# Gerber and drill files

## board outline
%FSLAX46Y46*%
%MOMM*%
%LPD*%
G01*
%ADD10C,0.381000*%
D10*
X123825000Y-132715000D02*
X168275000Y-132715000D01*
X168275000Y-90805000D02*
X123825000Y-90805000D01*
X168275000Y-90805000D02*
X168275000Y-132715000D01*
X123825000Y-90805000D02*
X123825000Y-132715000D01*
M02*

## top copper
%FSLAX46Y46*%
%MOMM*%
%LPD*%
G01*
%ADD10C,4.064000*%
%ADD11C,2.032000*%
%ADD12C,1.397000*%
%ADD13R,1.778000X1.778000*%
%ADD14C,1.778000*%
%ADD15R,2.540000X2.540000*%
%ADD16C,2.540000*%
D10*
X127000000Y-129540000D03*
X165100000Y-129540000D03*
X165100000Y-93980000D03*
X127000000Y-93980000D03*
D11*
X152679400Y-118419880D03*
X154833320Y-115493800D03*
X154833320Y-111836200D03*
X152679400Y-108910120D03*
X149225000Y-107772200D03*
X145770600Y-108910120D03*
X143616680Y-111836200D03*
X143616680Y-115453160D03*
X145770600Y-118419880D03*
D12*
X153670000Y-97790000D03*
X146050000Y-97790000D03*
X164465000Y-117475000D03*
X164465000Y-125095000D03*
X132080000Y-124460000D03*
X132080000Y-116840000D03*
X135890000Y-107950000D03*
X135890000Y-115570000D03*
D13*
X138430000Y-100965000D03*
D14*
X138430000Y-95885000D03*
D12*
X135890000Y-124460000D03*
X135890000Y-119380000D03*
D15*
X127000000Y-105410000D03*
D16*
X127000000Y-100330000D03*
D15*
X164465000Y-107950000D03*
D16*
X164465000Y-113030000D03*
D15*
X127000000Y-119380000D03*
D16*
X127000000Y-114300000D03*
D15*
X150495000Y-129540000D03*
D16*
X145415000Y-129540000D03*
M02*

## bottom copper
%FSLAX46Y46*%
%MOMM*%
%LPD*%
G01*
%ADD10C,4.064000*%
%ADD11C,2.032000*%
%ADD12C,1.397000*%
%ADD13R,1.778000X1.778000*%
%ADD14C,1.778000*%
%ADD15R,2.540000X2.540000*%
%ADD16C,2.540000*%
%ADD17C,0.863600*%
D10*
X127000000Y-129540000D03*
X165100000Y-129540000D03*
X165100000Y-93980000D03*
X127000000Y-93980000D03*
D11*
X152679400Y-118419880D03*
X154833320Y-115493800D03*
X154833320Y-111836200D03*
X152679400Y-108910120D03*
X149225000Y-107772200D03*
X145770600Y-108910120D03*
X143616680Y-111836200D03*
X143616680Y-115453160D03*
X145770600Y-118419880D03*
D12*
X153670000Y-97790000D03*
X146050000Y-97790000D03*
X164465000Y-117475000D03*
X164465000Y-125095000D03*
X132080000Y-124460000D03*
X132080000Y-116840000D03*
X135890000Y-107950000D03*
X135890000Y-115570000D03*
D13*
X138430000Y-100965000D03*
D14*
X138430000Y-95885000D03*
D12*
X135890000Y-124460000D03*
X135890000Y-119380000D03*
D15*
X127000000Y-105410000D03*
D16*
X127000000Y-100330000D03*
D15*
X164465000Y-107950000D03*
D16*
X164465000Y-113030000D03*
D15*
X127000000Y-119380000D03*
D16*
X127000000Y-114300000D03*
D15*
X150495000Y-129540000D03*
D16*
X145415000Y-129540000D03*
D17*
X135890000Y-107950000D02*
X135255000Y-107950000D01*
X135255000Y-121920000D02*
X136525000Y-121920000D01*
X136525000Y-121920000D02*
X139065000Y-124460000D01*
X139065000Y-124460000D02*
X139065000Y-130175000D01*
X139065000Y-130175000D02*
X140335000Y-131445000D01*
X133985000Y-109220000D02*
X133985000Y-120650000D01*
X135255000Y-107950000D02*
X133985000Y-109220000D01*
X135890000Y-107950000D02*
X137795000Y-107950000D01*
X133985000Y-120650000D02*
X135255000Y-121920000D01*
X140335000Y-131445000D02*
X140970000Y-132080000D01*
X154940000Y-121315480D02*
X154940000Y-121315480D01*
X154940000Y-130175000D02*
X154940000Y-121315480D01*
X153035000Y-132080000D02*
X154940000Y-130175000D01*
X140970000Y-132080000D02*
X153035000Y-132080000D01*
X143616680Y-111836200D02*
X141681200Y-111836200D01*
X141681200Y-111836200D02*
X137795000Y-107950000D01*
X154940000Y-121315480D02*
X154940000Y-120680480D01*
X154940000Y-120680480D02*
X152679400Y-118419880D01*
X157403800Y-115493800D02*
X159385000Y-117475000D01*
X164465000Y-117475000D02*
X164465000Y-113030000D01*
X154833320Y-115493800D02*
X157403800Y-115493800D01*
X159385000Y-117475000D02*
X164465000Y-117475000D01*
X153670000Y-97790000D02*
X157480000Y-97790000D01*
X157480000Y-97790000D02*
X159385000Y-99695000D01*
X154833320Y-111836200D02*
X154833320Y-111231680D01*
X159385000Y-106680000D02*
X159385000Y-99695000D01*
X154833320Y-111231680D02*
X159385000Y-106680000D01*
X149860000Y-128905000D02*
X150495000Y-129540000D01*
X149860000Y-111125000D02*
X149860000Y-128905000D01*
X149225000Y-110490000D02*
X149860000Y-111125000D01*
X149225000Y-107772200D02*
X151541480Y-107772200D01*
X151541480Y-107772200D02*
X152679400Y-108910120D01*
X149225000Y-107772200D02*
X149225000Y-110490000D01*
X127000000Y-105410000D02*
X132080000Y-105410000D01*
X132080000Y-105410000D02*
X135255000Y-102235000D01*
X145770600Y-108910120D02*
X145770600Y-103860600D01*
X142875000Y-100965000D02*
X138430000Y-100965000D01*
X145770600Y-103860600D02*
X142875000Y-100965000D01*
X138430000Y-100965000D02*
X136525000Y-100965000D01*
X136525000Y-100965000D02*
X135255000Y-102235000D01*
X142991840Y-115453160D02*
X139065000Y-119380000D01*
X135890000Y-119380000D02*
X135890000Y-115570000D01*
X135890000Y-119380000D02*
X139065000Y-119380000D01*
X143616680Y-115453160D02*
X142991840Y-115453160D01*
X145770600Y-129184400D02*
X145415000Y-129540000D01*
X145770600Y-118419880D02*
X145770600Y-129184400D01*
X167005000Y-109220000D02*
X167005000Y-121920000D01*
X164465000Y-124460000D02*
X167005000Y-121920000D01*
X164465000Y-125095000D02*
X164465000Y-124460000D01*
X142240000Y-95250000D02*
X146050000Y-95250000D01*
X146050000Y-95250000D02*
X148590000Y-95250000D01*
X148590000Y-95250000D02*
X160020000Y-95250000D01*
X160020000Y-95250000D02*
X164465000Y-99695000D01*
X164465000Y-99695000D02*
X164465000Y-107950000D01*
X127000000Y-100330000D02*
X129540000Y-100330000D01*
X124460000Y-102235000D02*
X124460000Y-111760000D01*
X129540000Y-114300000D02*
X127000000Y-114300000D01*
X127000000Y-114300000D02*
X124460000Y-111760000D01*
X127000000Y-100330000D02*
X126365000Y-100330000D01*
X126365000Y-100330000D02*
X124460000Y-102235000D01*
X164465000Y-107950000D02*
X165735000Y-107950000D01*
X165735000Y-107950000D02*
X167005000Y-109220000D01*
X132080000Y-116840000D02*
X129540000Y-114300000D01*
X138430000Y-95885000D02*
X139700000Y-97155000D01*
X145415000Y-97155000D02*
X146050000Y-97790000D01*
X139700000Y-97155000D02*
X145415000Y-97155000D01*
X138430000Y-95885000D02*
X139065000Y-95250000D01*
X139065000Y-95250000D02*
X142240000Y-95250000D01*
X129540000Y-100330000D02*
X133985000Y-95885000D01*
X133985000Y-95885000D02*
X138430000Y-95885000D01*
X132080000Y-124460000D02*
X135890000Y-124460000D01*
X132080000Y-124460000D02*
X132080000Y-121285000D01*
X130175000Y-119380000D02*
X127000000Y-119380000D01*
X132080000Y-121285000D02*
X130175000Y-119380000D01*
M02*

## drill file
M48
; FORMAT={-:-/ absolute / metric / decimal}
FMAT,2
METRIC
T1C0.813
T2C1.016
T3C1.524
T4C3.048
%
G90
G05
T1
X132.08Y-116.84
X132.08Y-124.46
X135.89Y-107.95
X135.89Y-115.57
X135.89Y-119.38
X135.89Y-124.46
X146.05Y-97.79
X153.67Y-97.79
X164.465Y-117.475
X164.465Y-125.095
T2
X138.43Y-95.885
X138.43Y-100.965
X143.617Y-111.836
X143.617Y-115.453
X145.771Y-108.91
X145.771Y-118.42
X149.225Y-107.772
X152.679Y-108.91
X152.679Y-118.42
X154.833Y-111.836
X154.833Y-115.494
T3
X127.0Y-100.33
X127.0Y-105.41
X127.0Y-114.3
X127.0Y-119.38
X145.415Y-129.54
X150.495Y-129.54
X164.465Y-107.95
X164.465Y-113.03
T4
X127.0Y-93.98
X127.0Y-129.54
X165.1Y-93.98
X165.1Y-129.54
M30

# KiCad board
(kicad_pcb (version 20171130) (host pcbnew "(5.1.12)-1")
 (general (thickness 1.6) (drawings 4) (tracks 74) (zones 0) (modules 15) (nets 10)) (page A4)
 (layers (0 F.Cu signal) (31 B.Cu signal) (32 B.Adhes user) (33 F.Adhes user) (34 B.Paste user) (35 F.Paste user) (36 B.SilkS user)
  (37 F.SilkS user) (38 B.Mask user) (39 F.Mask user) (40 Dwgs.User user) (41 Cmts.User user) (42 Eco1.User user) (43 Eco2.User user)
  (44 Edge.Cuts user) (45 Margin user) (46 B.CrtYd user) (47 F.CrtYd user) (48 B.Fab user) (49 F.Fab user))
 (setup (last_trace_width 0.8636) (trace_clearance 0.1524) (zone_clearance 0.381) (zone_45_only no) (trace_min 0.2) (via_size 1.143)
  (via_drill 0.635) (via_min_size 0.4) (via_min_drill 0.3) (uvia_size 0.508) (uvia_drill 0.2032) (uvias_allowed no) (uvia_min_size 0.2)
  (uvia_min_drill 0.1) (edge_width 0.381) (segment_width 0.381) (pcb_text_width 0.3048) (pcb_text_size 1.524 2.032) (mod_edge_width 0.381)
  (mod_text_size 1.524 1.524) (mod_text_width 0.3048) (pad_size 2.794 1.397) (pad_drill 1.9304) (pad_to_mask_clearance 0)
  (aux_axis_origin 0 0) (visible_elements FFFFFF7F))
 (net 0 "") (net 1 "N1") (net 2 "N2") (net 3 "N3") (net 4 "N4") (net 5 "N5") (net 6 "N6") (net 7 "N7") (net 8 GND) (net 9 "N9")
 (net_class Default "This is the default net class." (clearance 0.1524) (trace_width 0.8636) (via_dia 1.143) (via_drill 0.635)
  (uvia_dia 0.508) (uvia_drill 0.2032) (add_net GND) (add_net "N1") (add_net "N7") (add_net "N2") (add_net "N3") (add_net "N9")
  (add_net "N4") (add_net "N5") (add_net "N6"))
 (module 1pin (layer F.Cu) (at 127 129.54)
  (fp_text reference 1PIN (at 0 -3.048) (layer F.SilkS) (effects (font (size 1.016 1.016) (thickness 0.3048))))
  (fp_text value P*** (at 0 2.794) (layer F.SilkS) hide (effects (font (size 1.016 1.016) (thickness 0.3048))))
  (pad 1 thru_hole circle (at 0 0) (size 4.064 4.064) (drill 3.048) (layers *.Cu *.Mask F.SilkS)))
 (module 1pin (layer F.Cu) (at 165.1 129.54)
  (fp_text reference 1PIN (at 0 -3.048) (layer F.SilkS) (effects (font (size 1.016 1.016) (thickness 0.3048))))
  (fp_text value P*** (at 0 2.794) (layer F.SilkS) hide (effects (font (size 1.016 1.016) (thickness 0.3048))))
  (pad 1 thru_hole circle (at 0 0) (size 4.064 4.064) (drill 3.048) (layers *.Cu *.Mask F.SilkS)))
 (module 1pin (layer F.Cu) (at 165.1 93.98)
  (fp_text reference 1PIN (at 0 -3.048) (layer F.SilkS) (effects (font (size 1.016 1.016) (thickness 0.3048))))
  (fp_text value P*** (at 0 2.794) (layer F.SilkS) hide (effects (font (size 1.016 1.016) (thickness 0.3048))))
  (pad 1 thru_hole circle (at 0 0) (size 4.064 4.064) (drill 3.048) (layers *.Cu *.Mask F.SilkS)))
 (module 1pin (layer F.Cu) (at 127 93.98)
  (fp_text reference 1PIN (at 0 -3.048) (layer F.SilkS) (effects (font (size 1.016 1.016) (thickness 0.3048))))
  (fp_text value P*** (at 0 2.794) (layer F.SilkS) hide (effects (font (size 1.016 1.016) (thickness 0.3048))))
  (pad 1 thru_hole circle (at 0 0) (size 4.064 4.064) (drill 3.048) (layers *.Cu *.Mask F.SilkS)))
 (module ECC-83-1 (layer F.Cu) (at 149.225 113.665)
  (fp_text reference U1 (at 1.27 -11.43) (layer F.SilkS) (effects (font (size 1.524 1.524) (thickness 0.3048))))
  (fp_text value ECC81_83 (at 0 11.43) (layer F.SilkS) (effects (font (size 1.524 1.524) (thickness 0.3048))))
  (pad 1 thru_hole circle (at 3.4544 4.75488) (size 2.032 2.032) (drill 1.016) (layers *.Cu *.Mask F.SilkS) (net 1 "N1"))
  (pad 2 thru_hole circle (at 5.60832 1.8288) (size 2.032 2.032) (drill 1.016) (layers *.Cu *.Mask F.SilkS) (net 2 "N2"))
  (pad 3 thru_hole circle (at 5.60832 -1.8288) (size 2.032 2.032) (drill 1.016) (layers *.Cu *.Mask F.SilkS) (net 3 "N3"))
  (pad 4 thru_hole circle (at 3.4544 -4.75488) (size 2.032 2.032) (drill 1.016) (layers *.Cu *.Mask F.SilkS) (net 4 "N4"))
  (pad 5 thru_hole circle (at 0 -5.8928) (size 2.032 2.032) (drill 1.016) (layers *.Cu *.Mask F.SilkS) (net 4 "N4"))
  (pad 6 thru_hole circle (at -3.4544 -4.75488) (size 2.032 2.032) (drill 1.016) (layers *.Cu *.Mask F.SilkS) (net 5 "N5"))
  (pad 7 thru_hole circle (at -5.60832 -1.8288) (size 2.032 2.032) (drill 1.016) (layers *.Cu *.Mask F.SilkS) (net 1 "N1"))
  (pad 8 thru_hole circle (at -5.60832 1.78816) (size 2.032 2.032) (drill 1.016) (layers *.Cu *.Mask F.SilkS) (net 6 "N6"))
  (pad 9 thru_hole circle (at -3.4544 4.75488) (size 2.032 2.032) (drill 1.016) (layers *.Cu *.Mask F.SilkS) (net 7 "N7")))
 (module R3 (layer F.Cu) (at 149.86 97.79 180) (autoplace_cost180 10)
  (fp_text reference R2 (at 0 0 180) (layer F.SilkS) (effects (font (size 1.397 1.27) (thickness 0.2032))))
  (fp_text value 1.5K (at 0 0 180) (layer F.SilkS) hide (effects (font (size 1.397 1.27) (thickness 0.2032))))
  (pad 1 thru_hole circle (at -3.81 0 180) (size 1.397 1.397) (drill 0.8128) (layers *.Cu *.Mask F.SilkS) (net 3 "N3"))
  (pad 2 thru_hole circle (at 3.81 0 180) (size 1.397 1.397) (drill 0.8128) (layers *.Cu *.Mask F.SilkS) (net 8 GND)))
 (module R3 (layer F.Cu) (at 164.465 121.285 270) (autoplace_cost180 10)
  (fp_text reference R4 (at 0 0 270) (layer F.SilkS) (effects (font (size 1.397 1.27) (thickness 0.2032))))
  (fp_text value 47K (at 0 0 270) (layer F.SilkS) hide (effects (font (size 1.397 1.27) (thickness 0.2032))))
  (pad 1 thru_hole circle (at -3.81 0 270) (size 1.397 1.397) (drill 0.8128) (layers *.Cu *.Mask F.SilkS) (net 2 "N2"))
  (pad 2 thru_hole circle (at 3.81 0 270) (size 1.397 1.397) (drill 0.8128) (layers *.Cu *.Mask F.SilkS) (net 8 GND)))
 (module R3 (layer F.Cu) (at 132.08 120.65 90) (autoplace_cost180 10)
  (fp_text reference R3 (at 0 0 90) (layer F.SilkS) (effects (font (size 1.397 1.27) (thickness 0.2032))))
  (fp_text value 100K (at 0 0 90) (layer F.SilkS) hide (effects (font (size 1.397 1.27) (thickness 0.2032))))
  (pad 1 thru_hole circle (at -3.81 0 90) (size 1.397 1.397) (drill 0.8128) (layers *.Cu *.Mask F.SilkS) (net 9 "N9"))
  (pad 2 thru_hole circle (at 3.81 0 90) (size 1.397 1.397) (drill 0.8128) (layers *.Cu *.Mask F.SilkS) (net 8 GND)))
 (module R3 (layer F.Cu) (at 135.89 111.76 270) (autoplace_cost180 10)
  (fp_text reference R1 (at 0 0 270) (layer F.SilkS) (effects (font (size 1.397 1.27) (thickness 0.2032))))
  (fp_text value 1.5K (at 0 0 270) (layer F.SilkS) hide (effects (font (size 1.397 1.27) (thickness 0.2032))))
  (pad 1 thru_hole circle (at -3.81 0 270) (size 1.397 1.397) (drill 0.8128) (layers *.Cu *.Mask F.SilkS) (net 1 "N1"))
  (pad 2 thru_hole circle (at 3.81 0 270) (size 1.397 1.397) (drill 0.8128) (layers *.Cu *.Mask F.SilkS) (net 6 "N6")))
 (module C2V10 (layer F.Cu) (at 138.43 98.425 90)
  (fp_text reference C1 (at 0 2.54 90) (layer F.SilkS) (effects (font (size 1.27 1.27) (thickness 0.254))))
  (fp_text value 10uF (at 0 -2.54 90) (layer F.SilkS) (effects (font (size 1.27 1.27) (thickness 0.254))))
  (pad 1 thru_hole rect (at -2.54 0 90) (size 1.778 1.778) (drill 1.016) (layers *.Cu *.Mask F.SilkS) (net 5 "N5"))
  (pad 2 thru_hole circle (at 2.54 0 90) (size 1.778 1.778) (drill 1.016) (layers *.Cu *.Mask F.SilkS) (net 8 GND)))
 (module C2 (layer F.Cu) (at 135.89 121.92 90)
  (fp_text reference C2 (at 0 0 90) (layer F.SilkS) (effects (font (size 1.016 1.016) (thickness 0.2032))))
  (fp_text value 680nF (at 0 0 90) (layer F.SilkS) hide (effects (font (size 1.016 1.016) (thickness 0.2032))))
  (pad 1 thru_hole circle (at -2.54 0 90) (size 1.397 1.397) (drill 0.8128) (layers *.Cu *.Mask F.SilkS) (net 9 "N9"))
  (pad 2 thru_hole circle (at 2.54 0 90) (size 1.397 1.397) (drill 0.8128) (layers *.Cu *.Mask F.SilkS) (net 6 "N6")))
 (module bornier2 (layer F.Cu) (at 127 102.87 90)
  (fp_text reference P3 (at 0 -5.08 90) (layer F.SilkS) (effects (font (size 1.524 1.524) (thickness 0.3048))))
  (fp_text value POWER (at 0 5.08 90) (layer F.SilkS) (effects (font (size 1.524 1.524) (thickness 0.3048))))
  (pad 1 thru_hole rect (at -2.54 0 90) (size 2.54 2.54) (drill 1.524) (layers *.Cu *.Mask F.SilkS) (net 5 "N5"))
  (pad 2 thru_hole circle (at 2.54 0 90) (size 2.54 2.54) (drill 1.524) (layers *.Cu *.Mask F.SilkS) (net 8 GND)))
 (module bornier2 (layer F.Cu) (at 164.465 110.49 270)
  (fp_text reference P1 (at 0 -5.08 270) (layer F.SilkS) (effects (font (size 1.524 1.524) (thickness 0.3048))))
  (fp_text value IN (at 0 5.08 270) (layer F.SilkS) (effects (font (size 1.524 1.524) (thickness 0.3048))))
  (pad 1 thru_hole rect (at -2.54 0 270) (size 2.54 2.54) (drill 1.524) (layers *.Cu *.Mask F.SilkS) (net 8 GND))
  (pad 2 thru_hole circle (at 2.54 0 270) (size 2.54 2.54) (drill 1.524) (layers *.Cu *.Mask F.SilkS) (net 2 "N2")))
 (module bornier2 (layer F.Cu) (at 127 116.84 90)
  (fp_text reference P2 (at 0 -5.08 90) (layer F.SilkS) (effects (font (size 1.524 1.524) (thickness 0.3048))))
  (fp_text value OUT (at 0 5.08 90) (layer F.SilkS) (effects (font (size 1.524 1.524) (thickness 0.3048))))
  (pad 1 thru_hole rect (at -2.54 0 90) (size 2.54 2.54) (drill 1.524) (layers *.Cu *.Mask F.SilkS) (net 9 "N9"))
  (pad 2 thru_hole circle (at 2.54 0 90) (size 2.54 2.54) (drill 1.524) (layers *.Cu *.Mask F.SilkS) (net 8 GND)))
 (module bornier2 (layer F.Cu) (at 147.955 129.54 180)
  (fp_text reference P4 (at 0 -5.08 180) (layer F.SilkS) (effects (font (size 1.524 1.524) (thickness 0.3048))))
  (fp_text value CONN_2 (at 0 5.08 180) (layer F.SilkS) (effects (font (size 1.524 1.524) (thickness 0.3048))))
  (pad 1 thru_hole rect (at -2.54 0 180) (size 2.54 2.54) (drill 1.524) (layers *.Cu *.Mask F.SilkS) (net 4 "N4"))
  (pad 2 thru_hole circle (at 2.54 0 180) (size 2.54 2.54) (drill 1.524) (layers *.Cu *.Mask F.SilkS) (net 7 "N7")))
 (gr_line (start 123.825 132.715) (end 168.275 132.715) (angle 90) (layer Edge.Cuts) (width 0.381))
 (gr_line (start 168.275 90.805) (end 123.825 90.805) (angle 90) (layer Edge.Cuts) (width 0.381))
 (gr_line (start 168.275 90.805) (end 168.275 132.715) (angle 90) (layer Edge.Cuts) (width 0.381))
 (gr_line (start 123.825 90.805) (end 123.825 132.715) (angle 90) (layer Edge.Cuts) (width 0.381))
 (segment (start 135.89 107.95) (end 135.255 107.95) (width 0.8636) (layer B.Cu) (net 1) (status 800))
 (segment (start 135.255 121.92) (end 136.525 121.92) (width 0.8636) (layer B.Cu) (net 1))
 (segment (start 136.525 121.92) (end 139.065 124.46) (width 0.8636) (layer B.Cu) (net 1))
 (segment (start 139.065 124.46) (end 139.065 130.175) (width 0.8636) (layer B.Cu) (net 1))
 (segment (start 139.065 130.175) (end 140.335 131.445) (width 0.8636) (layer B.Cu) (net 1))
 (segment (start 133.985 109.22) (end 133.985 120.65) (width 0.8636) (layer B.Cu) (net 1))
 (segment (start 135.255 107.95) (end 133.985 109.22) (width 0.8636) (layer B.Cu) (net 1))
 (segment (start 135.89 107.95) (end 137.795 107.95) (width 0.8636) (layer B.Cu) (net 1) (status 800))
 (segment (start 133.985 120.65) (end 135.255 121.92) (width 0.8636) (layer B.Cu) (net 1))
 (segment (start 140.335 131.445) (end 140.97 132.08) (width 0.8636) (layer B.Cu) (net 1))
 (segment (start 154.94 121.31548) (end 154.94 121.31548) (width 0.8636) (layer B.Cu) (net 1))
 (segment (start 154.94 130.175) (end 154.94 121.31548) (width 0.8636) (layer B.Cu) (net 1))
 (segment (start 153.035 132.08) (end 154.94 130.175) (width 0.8636) (layer B.Cu) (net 1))
 (segment (start 140.97 132.08) (end 153.035 132.08) (width 0.8636) (layer B.Cu) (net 1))
 (segment (start 143.61668 111.8362) (end 141.6812 111.8362) (width 0.8636) (layer B.Cu) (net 1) (status 800))
 (segment (start 141.6812 111.8362) (end 137.795 107.95) (width 0.8636) (layer B.Cu) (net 1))
 (segment (start 154.94 121.31548) (end 154.94 120.68048) (width 0.8636) (layer B.Cu) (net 1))
 (segment (start 154.94 120.68048) (end 152.6794 118.41988) (width 0.8636) (layer B.Cu) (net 1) (status 400))
 (segment (start 157.4038 115.4938) (end 159.385 117.475) (width 0.8636) (layer B.Cu) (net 2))
 (segment (start 164.465 117.475) (end 164.465 113.03) (width 0.8636) (layer B.Cu) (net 2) (status C00))
 (segment (start 154.83332 115.4938) (end 157.4038 115.4938) (width 0.8636) (layer B.Cu) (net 2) (status 800))
 (segment (start 159.385 117.475) (end 164.465 117.475) (width 0.8636) (layer B.Cu) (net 2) (status 400))
 (segment (start 153.67 97.79) (end 157.48 97.79) (width 0.8636) (layer B.Cu) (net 3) (status 800))
 (segment (start 157.48 97.79) (end 159.385 99.695) (width 0.8636) (layer B.Cu) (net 3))
 (segment (start 154.83332 111.8362) (end 154.83332 111.23168) (width 0.8636) (layer B.Cu) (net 3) (status 800))
 (segment (start 159.385 106.68) (end 159.385 99.695) (width 0.8636) (layer B.Cu) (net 3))
 (segment (start 154.83332 111.23168) (end 159.385 106.68) (width 0.8636) (layer B.Cu) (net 3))
 (segment (start 149.86 128.905) (end 150.495 129.54) (width 0.8636) (layer B.Cu) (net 4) (status 400))
 (segment (start 149.86 111.125) (end 149.86 128.905) (width 0.8636) (layer B.Cu) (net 4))
 (segment (start 149.225 110.49) (end 149.86 111.125) (width 0.8636) (layer B.Cu) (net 4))
 (segment (start 149.225 107.7722) (end 151.54148 107.7722) (width 0.8636) (layer B.Cu) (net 4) (status 800))
 (segment (start 151.54148 107.7722) (end 152.6794 108.91012) (width 0.8636) (layer B.Cu) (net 4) (status 400))
 (segment (start 149.225 107.7722) (end 149.225 110.49) (width 0.8636) (layer B.Cu) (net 4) (status 800))
 (segment (start 127 105.41) (end 132.08 105.41) (width 0.8636) (layer B.Cu) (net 5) (status 800))
 (segment (start 132.08 105.41) (end 135.255 102.235) (width 0.8636) (layer B.Cu) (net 5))
 (segment (start 145.7706 108.91012) (end 145.7706 103.8606) (width 0.8636) (layer B.Cu) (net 5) (status 800))
 (segment (start 142.875 100.965) (end 138.43 100.965) (width 0.8636) (layer B.Cu) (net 5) (status 400))
 (segment (start 145.7706 103.8606) (end 142.875 100.965) (width 0.8636) (layer B.Cu) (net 5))
 (segment (start 138.43 100.965) (end 136.525 100.965) (width 0.8636) (layer B.Cu) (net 5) (status 800))
 (segment (start 136.525 100.965) (end 135.255 102.235) (width 0.8636) (layer B.Cu) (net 5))
 (segment (start 142.99184 115.45316) (end 139.065 119.38) (width 0.8636) (layer B.Cu) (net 6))
 (segment (start 135.89 119.38) (end 135.89 115.57) (width 0.8636) (layer B.Cu) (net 6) (status C00))
 (segment (start 135.89 119.38) (end 139.065 119.38) (width 0.8636) (layer B.Cu) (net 6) (status 800))
 (segment (start 143.61668 115.45316) (end 142.99184 115.45316) (width 0.8636) (layer B.Cu) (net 6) (status 800))
 (segment (start 145.7706 129.1844) (end 145.415 129.54) (width 0.8636) (layer B.Cu) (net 7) (status 400))
 (segment (start 145.7706 118.41988) (end 145.7706 129.1844) (width 0.8636) (layer B.Cu) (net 7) (status 800))
 (segment (start 167.005 109.22) (end 167.005 121.92) (width 0.8636) (layer B.Cu) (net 8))
 (segment (start 164.465 124.46) (end 167.005 121.92) (width 0.8636) (layer B.Cu) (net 8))
 (segment (start 164.465 125.095) (end 164.465 124.46) (width 0.8636) (layer B.Cu) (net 8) (status 800))
 (segment (start 142.24 95.25) (end 146.05 95.25) (width 0.8636) (layer B.Cu) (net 8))
 (segment (start 146.05 95.25) (end 148.59 95.25) (width 0.8636) (layer B.Cu) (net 8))
 (segment (start 148.59 95.25) (end 160.02 95.25) (width 0.8636) (layer B.Cu) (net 8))
 (segment (start 160.02 95.25) (end 164.465 99.695) (width 0.8636) (layer B.Cu) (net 8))
 (segment (start 164.465 99.695) (end 164.465 107.95) (width 0.8636) (layer B.Cu) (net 8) (status 400))
 (segment (start 127 100.33) (end 129.54 100.33) (width 0.8636) (layer B.Cu) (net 8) (status 800))
 (segment (start 124.46 102.235) (end 124.46 111.76) (width 0.8636) (layer B.Cu) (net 8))
 (segment (start 129.54 114.3) (end 127 114.3) (width 0.8636) (layer B.Cu) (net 8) (status 400))
 (segment (start 127 114.3) (end 124.46 111.76) (width 0.8636) (layer B.Cu) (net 8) (status 800))
 (segment (start 127 100.33) (end 126.365 100.33) (width 0.8636) (layer B.Cu) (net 8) (status 800))
 (segment (start 126.365 100.33) (end 124.46 102.235) (width 0.8636) (layer B.Cu) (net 8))
 (segment (start 164.465 107.95) (end 165.735 107.95) (width 0.8636) (layer B.Cu) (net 8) (status 800))
 (segment (start 165.735 107.95) (end 167.005 109.22) (width 0.8636) (layer B.Cu) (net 8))
 (segment (start 132.08 116.84) (end 129.54 114.3) (width 0.8636) (layer B.Cu) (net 8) (status 800))
 (segment (start 138.43 95.885) (end 139.7 97.155) (width 0.8636) (layer B.Cu) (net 8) (status 800))
 (segment (start 145.415 97.155) (end 146.05 97.79) (width 0.8636) (layer B.Cu) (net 8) (status 400))
 (segment (start 139.7 97.155) (end 145.415 97.155) (width 0.8636) (layer B.Cu) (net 8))
 (segment (start 138.43 95.885) (end 139.065 95.25) (width 0.8636) (layer B.Cu) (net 8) (status 800))
 (segment (start 139.065 95.25) (end 142.24 95.25) (width 0.8636) (layer B.Cu) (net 8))
 (segment (start 129.54 100.33) (end 133.985 95.885) (width 0.8636) (layer B.Cu) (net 8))
 (segment (start 133.985 95.885) (end 138.43 95.885) (width 0.8636) (layer B.Cu) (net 8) (status 400))
 (segment (start 132.08 124.46) (end 135.89 124.46) (width 0.8636) (layer B.Cu) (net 9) (status C00))
 (segment (start 132.08 124.46) (end 132.08 121.285) (width 0.8636) (layer B.Cu) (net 9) (status 800))
 (segment (start 130.175 119.38) (end 127 119.38) (width 0.8636) (layer B.Cu) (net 9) (status 400))
 (segment (start 132.08 121.285) (end 130.175 119.38) (width 0.8636) (layer B.Cu) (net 9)))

